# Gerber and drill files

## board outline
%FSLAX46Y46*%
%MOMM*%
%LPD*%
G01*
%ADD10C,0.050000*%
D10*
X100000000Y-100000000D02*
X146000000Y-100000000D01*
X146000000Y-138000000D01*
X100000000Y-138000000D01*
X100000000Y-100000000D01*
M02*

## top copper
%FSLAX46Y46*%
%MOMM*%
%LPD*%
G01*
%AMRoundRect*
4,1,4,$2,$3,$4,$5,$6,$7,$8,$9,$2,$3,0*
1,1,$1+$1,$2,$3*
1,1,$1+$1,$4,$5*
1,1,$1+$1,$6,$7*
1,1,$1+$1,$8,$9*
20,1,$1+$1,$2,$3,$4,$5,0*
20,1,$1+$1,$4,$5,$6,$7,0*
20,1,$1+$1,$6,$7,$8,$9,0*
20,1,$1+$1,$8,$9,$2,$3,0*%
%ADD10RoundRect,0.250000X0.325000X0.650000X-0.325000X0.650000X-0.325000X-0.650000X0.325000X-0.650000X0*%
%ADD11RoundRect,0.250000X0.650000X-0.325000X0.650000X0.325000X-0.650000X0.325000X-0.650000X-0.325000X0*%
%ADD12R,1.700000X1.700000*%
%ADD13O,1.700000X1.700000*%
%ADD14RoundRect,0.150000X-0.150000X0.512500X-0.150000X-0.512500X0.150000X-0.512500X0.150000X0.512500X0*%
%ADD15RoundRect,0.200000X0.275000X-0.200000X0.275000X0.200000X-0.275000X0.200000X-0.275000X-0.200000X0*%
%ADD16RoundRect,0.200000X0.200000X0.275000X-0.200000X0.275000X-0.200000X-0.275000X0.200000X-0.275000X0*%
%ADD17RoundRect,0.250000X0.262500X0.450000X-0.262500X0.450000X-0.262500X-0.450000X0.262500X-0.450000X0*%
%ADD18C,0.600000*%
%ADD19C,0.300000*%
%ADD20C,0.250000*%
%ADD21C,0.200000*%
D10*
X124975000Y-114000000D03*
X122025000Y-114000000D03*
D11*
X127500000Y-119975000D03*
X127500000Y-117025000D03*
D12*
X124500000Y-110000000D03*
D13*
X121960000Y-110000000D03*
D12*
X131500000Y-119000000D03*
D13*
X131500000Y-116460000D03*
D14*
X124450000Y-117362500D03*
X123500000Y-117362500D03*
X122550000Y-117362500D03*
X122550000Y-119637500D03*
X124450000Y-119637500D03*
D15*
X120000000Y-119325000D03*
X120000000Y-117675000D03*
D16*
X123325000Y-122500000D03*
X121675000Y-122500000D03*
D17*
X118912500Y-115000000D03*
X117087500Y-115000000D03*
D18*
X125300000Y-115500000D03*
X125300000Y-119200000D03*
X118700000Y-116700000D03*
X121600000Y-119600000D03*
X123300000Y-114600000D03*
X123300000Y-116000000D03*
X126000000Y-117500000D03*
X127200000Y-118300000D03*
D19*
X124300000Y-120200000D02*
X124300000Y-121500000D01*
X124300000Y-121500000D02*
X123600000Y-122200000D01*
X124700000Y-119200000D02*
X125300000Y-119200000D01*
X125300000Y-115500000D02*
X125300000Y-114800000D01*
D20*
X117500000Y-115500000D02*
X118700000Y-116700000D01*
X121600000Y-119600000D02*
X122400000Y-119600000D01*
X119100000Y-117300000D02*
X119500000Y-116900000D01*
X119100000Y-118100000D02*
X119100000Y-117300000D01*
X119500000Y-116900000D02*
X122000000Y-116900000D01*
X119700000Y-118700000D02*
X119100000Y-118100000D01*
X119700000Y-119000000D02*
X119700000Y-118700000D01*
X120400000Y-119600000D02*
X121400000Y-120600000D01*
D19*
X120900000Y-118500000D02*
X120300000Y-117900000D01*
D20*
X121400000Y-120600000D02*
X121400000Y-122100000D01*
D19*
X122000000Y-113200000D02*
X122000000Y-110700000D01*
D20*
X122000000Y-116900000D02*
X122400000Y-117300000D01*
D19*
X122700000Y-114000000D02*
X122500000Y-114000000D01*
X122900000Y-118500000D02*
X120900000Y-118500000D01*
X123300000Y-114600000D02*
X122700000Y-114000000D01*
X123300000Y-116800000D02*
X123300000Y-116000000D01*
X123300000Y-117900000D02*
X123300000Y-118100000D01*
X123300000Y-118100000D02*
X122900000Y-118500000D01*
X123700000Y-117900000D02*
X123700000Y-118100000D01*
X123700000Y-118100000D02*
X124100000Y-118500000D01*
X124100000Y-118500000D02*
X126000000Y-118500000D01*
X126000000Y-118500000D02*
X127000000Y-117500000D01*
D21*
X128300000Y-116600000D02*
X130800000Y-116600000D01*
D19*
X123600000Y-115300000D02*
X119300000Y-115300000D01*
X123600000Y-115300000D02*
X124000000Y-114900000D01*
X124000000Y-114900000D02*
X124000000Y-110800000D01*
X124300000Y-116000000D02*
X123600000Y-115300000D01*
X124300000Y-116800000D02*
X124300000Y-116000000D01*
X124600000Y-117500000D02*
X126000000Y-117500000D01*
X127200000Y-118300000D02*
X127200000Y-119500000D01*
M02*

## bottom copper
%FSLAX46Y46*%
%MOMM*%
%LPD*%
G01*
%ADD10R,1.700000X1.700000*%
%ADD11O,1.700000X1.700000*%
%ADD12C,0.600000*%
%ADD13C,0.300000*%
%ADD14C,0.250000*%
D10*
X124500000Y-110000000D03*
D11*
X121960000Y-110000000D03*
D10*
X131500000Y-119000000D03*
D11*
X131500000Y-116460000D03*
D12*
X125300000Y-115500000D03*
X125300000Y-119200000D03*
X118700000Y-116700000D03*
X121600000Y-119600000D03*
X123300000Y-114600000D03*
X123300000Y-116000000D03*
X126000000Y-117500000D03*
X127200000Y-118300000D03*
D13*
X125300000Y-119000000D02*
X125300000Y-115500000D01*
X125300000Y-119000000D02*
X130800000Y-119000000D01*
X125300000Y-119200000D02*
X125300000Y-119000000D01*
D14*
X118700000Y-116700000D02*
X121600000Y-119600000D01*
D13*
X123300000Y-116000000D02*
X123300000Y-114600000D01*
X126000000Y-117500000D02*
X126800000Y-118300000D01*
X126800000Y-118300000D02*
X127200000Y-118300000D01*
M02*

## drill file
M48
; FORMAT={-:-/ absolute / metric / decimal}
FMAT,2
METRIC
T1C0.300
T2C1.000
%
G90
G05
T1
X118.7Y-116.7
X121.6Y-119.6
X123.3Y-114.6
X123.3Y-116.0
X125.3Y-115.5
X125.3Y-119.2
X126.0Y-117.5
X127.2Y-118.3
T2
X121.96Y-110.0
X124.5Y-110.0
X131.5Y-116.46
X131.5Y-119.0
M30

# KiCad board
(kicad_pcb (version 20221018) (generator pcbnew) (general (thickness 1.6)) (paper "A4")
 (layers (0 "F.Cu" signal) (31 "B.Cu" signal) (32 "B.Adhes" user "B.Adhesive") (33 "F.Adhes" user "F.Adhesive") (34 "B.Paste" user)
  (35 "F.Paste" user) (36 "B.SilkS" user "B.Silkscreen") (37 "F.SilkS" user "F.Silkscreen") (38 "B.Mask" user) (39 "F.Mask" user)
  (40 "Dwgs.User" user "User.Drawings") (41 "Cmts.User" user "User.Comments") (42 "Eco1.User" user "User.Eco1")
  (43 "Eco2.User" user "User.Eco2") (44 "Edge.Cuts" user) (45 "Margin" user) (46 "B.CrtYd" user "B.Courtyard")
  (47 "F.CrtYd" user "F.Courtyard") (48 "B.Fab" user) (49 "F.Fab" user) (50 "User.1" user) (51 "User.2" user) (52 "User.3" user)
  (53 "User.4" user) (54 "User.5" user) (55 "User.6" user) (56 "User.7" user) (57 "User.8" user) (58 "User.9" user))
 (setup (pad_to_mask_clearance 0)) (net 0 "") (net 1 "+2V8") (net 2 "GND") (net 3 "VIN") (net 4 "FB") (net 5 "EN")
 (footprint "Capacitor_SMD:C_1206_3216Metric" (layer "F.Cu") (at 123.5 114 180)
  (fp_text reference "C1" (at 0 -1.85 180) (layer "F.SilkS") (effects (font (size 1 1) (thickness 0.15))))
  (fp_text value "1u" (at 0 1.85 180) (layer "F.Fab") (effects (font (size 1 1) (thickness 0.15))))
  (pad "1" smd roundrect (at -1.475 0 180) (size 1.15 1.8) (layers "F.Cu" "F.Paste" "F.Mask") (roundrect_rratio 0.217391) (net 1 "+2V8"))
  (pad "2" smd roundrect (at 1.475 0 180) (size 1.15 1.8) (layers "F.Cu" "F.Paste" "F.Mask") (roundrect_rratio 0.217391) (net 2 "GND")))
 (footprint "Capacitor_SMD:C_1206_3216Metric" (layer "F.Cu") (at 127.5 118.5 90)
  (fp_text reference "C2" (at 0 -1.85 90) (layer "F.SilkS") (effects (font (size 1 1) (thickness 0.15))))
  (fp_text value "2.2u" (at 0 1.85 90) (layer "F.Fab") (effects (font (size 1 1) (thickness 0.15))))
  (pad "1" smd roundrect (at -1.475 0 90) (size 1.15 1.8) (layers "F.Cu" "F.Paste" "F.Mask") (roundrect_rratio 0.217391) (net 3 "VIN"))
  (pad "2" smd roundrect (at 1.475 0 90) (size 1.15 1.8) (layers "F.Cu" "F.Paste" "F.Mask") (roundrect_rratio 0.217391) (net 2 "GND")))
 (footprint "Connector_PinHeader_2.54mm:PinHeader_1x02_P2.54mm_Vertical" (layer "F.Cu") (at 124.5 110 -90)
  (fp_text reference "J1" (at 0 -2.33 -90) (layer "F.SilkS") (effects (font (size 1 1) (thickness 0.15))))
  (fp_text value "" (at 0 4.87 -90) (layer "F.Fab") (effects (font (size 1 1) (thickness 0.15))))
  (pad "1" thru_hole rect (at 0 0 270) (size 1.7 1.7) (drill 1) (layers "*.Cu" "*.Mask") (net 3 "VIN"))
  (pad "2" thru_hole oval (at 0 2.54 270) (size 1.7 1.7) (drill 1) (layers "*.Cu" "*.Mask") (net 2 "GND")))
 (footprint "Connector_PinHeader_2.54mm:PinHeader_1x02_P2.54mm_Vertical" (layer "F.Cu") (at 131.5 119 180)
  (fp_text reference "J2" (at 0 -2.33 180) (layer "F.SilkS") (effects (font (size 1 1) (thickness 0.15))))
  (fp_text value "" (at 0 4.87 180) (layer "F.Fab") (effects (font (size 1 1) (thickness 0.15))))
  (pad "1" thru_hole rect (at 0 0 180) (size 1.7 1.7) (drill 1) (layers "*.Cu" "*.Mask") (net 1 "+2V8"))
  (pad "2" thru_hole oval (at 0 2.54 180) (size 1.7 1.7) (drill 1) (layers "*.Cu" "*.Mask") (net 2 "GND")))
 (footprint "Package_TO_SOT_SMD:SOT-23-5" (layer "F.Cu") (at 123.5 118.5 -90)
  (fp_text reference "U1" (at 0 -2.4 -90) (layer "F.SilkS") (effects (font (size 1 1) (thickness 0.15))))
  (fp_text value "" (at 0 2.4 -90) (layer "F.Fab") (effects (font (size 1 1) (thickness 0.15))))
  (pad "1" smd roundrect (at -1.1375 -0.95 270) (size 1.325 0.6) (layers "F.Cu" "F.Paste" "F.Mask") (roundrect_rratio 0.25) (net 3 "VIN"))
  (pad "2" smd roundrect (at -1.1375 0 270) (size 1.325 0.6) (layers "F.Cu" "F.Paste" "F.Mask") (roundrect_rratio 0.25) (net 2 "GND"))
  (pad "3" smd roundrect (at -1.1375 0.95 270) (size 1.325 0.6) (layers "F.Cu" "F.Paste" "F.Mask") (roundrect_rratio 0.25) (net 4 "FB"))
  (pad "4" smd roundrect (at 1.1375 0.95 270) (size 1.325 0.6) (layers "F.Cu" "F.Paste" "F.Mask") (roundrect_rratio 0.25) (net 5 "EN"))
  (pad "5" smd roundrect (at 1.1375 -0.95 270) (size 1.325 0.6) (layers "F.Cu" "F.Paste" "F.Mask") (roundrect_rratio 0.25) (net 1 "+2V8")))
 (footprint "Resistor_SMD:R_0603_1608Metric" (layer "F.Cu") (at 120 118.5 90)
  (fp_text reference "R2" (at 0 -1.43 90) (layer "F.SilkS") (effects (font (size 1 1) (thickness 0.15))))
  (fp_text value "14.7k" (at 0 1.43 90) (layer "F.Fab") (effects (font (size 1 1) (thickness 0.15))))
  (pad "1" smd roundrect (at -0.825 0 90) (size 0.8 0.95) (layers "F.Cu" "F.Paste" "F.Mask") (roundrect_rratio 0.25) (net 4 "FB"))
  (pad "2" smd roundrect (at 0.825 0 90) (size 0.8 0.95) (layers "F.Cu" "F.Paste" "F.Mask") (roundrect_rratio 0.25) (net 2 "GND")))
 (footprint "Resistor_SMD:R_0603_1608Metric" (layer "F.Cu") (at 122.5 122.5 180)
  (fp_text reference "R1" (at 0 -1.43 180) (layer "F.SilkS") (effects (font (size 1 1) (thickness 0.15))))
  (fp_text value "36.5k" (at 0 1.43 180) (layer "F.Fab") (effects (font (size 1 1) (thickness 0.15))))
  (pad "1" smd roundrect (at -0.825 0 180) (size 0.8 0.95) (layers "F.Cu" "F.Paste" "F.Mask") (roundrect_rratio 0.25) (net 1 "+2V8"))
  (pad "2" smd roundrect (at 0.825 0 180) (size 0.8 0.95) (layers "F.Cu" "F.Paste" "F.Mask") (roundrect_rratio 0.25) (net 4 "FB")))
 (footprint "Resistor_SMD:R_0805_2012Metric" (layer "F.Cu") (at 118 115 180)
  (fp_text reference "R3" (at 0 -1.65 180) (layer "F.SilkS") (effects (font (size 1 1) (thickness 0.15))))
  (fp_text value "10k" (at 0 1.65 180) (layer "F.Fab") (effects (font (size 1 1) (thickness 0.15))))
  (pad "1" smd roundrect (at -0.9125 0 180) (size 1.025 1.4) (layers "F.Cu" "F.Paste" "F.Mask") (roundrect_rratio 0.243902) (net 3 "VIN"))
  (pad "2" smd roundrect (at 0.9125 0 180) (size 1.025 1.4) (layers "F.Cu" "F.Paste" "F.Mask") (roundrect_rratio 0.243902) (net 5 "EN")))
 (gr_rect (start 100 100) (end 146 138) (stroke (width 0.05) (type default)) (fill none) (layer "Edge.Cuts"))
 (segment (start 124.3 120.2) (end 124.3 121.5) (width 0.3) (layer "F.Cu") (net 1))
 (segment (start 124.3 121.5) (end 123.6 122.2) (width 0.3) (layer "F.Cu") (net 1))
 (segment (start 124.7 119.2) (end 125.3 119.2) (width 0.3) (layer "F.Cu") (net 1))
 (segment (start 125.3 115.5) (end 125.3 114.8) (width 0.3) (layer "F.Cu") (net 1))
 (via (at 125.3 115.5) (size 0.6) (drill 0.3) (layers "F.Cu" "B.Cu") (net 1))
 (via (at 125.3 119.2) (size 0.6) (drill 0.3) (layers "F.Cu" "B.Cu") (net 1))
 (segment (start 117.5 115.5) (end 118.7 116.7) (width 0.25) (layer "F.Cu") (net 5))
 (segment (start 121.6 119.6) (end 122.4 119.6) (width 0.25) (layer "F.Cu") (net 5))
 (segment (start 125.3 119) (end 125.3 115.5) (width 0.3) (layer "B.Cu") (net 1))
 (segment (start 125.3 119) (end 130.8 119) (width 0.3) (layer "B.Cu") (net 1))
 (segment (start 125.3 119.2) (end 125.3 119) (width 0.3) (layer "B.Cu") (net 1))
 (via (at 118.7 116.7) (size 0.6) (drill 0.3) (layers "F.Cu" "B.Cu") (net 5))
 (via (at 121.6 119.6) (size 0.6) (drill 0.3) (layers "F.Cu" "B.Cu") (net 5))
 (segment (start 118.7 116.7) (end 121.6 119.6) (width 0.25) (layer "B.Cu") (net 5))
 (segment (start 119.1 117.3) (end 119.5 116.9) (width 0.25) (layer "F.Cu") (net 4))
 (segment (start 119.1 118.1) (end 119.1 117.3) (width 0.25) (layer "F.Cu") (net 4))
 (segment (start 119.5 116.9) (end 122 116.9) (width 0.25) (layer "F.Cu") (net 4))
 (segment (start 119.7 118.7) (end 119.1 118.1) (width 0.25) (layer "F.Cu") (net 4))
 (segment (start 119.7 119) (end 119.7 118.7) (width 0.25) (layer "F.Cu") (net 4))
 (segment (start 120.4 119.6) (end 121.4 120.6) (width 0.25) (layer "F.Cu") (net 4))
 (segment (start 120.9 118.5) (end 120.3 117.9) (width 0.3) (layer "F.Cu") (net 2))
 (segment (start 121.4 120.6) (end 121.4 122.1) (width 0.25) (layer "F.Cu") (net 4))
 (segment (start 122 113.2) (end 122 110.7) (width 0.3) (layer "F.Cu") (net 2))
 (segment (start 122 116.9) (end 122.4 117.3) (width 0.25) (layer "F.Cu") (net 4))
 (segment (start 122.7 114) (end 122.5 114) (width 0.3) (layer "F.Cu") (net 2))
 (segment (start 122.9 118.5) (end 120.9 118.5) (width 0.3) (layer "F.Cu") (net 2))
 (segment (start 123.3 114.6) (end 122.7 114) (width 0.3) (layer "F.Cu") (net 2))
 (segment (start 123.3 116.8) (end 123.3 116) (width 0.3) (layer "F.Cu") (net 2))
 (segment (start 123.3 117.9) (end 123.3 118.1) (width 0.3) (layer "F.Cu") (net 2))
 (segment (start 123.3 118.1) (end 122.9 118.5) (width 0.3) (layer "F.Cu") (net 2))
 (segment (start 123.7 117.9) (end 123.7 118.1) (width 0.3) (layer "F.Cu") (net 2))
 (segment (start 123.7 118.1) (end 124.1 118.5) (width 0.3) (layer "F.Cu") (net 2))
 (segment (start 124.1 118.5) (end 126 118.5) (width 0.3) (layer "F.Cu") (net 2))
 (segment (start 126 118.5) (end 127 117.5) (width 0.3) (layer "F.Cu") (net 2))
 (segment (start 128.3 116.6) (end 130.8 116.6) (width 0.2) (layer "F.Cu") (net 2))
 (via (at 123.3 114.6) (size 0.6) (drill 0.3) (layers "F.Cu" "B.Cu") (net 2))
 (via (at 123.3 116) (size 0.6) (drill 0.3) (layers "F.Cu" "B.Cu") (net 2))
 (segment (start 123.3 116) (end 123.3 114.6) (width 0.3) (layer "B.Cu") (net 2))
 (segment (start 123.6 115.3) (end 119.3 115.3) (width 0.3) (layer "F.Cu") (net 3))
 (segment (start 123.6 115.3) (end 124 114.9) (width 0.3) (layer "F.Cu") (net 3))
 (segment (start 124 114.9) (end 124 110.8) (width 0.3) (layer "F.Cu") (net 3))
 (segment (start 124.3 116) (end 123.6 115.3) (width 0.3) (layer "F.Cu") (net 3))
 (segment (start 124.3 116.8) (end 124.3 116) (width 0.3) (layer "F.Cu") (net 3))
 (segment (start 124.6 117.5) (end 126 117.5) (width 0.3) (layer "F.Cu") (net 3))
 (segment (start 127.2 118.3) (end 127.2 119.5) (width 0.3) (layer "F.Cu") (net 3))
 (via (at 126 117.5) (size 0.6) (drill 0.3) (layers "F.Cu" "B.Cu") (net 3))
 (via (at 127.2 118.3) (size 0.6) (drill 0.3) (layers "F.Cu" "B.Cu") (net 3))
 (segment (start 126 117.5) (end 126.8 118.3) (width 0.3) (layer "B.Cu") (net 3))
 (segment (start 126.8 118.3) (end 127.2 118.3) (width 0.3) (layer "B.Cu") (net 3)))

